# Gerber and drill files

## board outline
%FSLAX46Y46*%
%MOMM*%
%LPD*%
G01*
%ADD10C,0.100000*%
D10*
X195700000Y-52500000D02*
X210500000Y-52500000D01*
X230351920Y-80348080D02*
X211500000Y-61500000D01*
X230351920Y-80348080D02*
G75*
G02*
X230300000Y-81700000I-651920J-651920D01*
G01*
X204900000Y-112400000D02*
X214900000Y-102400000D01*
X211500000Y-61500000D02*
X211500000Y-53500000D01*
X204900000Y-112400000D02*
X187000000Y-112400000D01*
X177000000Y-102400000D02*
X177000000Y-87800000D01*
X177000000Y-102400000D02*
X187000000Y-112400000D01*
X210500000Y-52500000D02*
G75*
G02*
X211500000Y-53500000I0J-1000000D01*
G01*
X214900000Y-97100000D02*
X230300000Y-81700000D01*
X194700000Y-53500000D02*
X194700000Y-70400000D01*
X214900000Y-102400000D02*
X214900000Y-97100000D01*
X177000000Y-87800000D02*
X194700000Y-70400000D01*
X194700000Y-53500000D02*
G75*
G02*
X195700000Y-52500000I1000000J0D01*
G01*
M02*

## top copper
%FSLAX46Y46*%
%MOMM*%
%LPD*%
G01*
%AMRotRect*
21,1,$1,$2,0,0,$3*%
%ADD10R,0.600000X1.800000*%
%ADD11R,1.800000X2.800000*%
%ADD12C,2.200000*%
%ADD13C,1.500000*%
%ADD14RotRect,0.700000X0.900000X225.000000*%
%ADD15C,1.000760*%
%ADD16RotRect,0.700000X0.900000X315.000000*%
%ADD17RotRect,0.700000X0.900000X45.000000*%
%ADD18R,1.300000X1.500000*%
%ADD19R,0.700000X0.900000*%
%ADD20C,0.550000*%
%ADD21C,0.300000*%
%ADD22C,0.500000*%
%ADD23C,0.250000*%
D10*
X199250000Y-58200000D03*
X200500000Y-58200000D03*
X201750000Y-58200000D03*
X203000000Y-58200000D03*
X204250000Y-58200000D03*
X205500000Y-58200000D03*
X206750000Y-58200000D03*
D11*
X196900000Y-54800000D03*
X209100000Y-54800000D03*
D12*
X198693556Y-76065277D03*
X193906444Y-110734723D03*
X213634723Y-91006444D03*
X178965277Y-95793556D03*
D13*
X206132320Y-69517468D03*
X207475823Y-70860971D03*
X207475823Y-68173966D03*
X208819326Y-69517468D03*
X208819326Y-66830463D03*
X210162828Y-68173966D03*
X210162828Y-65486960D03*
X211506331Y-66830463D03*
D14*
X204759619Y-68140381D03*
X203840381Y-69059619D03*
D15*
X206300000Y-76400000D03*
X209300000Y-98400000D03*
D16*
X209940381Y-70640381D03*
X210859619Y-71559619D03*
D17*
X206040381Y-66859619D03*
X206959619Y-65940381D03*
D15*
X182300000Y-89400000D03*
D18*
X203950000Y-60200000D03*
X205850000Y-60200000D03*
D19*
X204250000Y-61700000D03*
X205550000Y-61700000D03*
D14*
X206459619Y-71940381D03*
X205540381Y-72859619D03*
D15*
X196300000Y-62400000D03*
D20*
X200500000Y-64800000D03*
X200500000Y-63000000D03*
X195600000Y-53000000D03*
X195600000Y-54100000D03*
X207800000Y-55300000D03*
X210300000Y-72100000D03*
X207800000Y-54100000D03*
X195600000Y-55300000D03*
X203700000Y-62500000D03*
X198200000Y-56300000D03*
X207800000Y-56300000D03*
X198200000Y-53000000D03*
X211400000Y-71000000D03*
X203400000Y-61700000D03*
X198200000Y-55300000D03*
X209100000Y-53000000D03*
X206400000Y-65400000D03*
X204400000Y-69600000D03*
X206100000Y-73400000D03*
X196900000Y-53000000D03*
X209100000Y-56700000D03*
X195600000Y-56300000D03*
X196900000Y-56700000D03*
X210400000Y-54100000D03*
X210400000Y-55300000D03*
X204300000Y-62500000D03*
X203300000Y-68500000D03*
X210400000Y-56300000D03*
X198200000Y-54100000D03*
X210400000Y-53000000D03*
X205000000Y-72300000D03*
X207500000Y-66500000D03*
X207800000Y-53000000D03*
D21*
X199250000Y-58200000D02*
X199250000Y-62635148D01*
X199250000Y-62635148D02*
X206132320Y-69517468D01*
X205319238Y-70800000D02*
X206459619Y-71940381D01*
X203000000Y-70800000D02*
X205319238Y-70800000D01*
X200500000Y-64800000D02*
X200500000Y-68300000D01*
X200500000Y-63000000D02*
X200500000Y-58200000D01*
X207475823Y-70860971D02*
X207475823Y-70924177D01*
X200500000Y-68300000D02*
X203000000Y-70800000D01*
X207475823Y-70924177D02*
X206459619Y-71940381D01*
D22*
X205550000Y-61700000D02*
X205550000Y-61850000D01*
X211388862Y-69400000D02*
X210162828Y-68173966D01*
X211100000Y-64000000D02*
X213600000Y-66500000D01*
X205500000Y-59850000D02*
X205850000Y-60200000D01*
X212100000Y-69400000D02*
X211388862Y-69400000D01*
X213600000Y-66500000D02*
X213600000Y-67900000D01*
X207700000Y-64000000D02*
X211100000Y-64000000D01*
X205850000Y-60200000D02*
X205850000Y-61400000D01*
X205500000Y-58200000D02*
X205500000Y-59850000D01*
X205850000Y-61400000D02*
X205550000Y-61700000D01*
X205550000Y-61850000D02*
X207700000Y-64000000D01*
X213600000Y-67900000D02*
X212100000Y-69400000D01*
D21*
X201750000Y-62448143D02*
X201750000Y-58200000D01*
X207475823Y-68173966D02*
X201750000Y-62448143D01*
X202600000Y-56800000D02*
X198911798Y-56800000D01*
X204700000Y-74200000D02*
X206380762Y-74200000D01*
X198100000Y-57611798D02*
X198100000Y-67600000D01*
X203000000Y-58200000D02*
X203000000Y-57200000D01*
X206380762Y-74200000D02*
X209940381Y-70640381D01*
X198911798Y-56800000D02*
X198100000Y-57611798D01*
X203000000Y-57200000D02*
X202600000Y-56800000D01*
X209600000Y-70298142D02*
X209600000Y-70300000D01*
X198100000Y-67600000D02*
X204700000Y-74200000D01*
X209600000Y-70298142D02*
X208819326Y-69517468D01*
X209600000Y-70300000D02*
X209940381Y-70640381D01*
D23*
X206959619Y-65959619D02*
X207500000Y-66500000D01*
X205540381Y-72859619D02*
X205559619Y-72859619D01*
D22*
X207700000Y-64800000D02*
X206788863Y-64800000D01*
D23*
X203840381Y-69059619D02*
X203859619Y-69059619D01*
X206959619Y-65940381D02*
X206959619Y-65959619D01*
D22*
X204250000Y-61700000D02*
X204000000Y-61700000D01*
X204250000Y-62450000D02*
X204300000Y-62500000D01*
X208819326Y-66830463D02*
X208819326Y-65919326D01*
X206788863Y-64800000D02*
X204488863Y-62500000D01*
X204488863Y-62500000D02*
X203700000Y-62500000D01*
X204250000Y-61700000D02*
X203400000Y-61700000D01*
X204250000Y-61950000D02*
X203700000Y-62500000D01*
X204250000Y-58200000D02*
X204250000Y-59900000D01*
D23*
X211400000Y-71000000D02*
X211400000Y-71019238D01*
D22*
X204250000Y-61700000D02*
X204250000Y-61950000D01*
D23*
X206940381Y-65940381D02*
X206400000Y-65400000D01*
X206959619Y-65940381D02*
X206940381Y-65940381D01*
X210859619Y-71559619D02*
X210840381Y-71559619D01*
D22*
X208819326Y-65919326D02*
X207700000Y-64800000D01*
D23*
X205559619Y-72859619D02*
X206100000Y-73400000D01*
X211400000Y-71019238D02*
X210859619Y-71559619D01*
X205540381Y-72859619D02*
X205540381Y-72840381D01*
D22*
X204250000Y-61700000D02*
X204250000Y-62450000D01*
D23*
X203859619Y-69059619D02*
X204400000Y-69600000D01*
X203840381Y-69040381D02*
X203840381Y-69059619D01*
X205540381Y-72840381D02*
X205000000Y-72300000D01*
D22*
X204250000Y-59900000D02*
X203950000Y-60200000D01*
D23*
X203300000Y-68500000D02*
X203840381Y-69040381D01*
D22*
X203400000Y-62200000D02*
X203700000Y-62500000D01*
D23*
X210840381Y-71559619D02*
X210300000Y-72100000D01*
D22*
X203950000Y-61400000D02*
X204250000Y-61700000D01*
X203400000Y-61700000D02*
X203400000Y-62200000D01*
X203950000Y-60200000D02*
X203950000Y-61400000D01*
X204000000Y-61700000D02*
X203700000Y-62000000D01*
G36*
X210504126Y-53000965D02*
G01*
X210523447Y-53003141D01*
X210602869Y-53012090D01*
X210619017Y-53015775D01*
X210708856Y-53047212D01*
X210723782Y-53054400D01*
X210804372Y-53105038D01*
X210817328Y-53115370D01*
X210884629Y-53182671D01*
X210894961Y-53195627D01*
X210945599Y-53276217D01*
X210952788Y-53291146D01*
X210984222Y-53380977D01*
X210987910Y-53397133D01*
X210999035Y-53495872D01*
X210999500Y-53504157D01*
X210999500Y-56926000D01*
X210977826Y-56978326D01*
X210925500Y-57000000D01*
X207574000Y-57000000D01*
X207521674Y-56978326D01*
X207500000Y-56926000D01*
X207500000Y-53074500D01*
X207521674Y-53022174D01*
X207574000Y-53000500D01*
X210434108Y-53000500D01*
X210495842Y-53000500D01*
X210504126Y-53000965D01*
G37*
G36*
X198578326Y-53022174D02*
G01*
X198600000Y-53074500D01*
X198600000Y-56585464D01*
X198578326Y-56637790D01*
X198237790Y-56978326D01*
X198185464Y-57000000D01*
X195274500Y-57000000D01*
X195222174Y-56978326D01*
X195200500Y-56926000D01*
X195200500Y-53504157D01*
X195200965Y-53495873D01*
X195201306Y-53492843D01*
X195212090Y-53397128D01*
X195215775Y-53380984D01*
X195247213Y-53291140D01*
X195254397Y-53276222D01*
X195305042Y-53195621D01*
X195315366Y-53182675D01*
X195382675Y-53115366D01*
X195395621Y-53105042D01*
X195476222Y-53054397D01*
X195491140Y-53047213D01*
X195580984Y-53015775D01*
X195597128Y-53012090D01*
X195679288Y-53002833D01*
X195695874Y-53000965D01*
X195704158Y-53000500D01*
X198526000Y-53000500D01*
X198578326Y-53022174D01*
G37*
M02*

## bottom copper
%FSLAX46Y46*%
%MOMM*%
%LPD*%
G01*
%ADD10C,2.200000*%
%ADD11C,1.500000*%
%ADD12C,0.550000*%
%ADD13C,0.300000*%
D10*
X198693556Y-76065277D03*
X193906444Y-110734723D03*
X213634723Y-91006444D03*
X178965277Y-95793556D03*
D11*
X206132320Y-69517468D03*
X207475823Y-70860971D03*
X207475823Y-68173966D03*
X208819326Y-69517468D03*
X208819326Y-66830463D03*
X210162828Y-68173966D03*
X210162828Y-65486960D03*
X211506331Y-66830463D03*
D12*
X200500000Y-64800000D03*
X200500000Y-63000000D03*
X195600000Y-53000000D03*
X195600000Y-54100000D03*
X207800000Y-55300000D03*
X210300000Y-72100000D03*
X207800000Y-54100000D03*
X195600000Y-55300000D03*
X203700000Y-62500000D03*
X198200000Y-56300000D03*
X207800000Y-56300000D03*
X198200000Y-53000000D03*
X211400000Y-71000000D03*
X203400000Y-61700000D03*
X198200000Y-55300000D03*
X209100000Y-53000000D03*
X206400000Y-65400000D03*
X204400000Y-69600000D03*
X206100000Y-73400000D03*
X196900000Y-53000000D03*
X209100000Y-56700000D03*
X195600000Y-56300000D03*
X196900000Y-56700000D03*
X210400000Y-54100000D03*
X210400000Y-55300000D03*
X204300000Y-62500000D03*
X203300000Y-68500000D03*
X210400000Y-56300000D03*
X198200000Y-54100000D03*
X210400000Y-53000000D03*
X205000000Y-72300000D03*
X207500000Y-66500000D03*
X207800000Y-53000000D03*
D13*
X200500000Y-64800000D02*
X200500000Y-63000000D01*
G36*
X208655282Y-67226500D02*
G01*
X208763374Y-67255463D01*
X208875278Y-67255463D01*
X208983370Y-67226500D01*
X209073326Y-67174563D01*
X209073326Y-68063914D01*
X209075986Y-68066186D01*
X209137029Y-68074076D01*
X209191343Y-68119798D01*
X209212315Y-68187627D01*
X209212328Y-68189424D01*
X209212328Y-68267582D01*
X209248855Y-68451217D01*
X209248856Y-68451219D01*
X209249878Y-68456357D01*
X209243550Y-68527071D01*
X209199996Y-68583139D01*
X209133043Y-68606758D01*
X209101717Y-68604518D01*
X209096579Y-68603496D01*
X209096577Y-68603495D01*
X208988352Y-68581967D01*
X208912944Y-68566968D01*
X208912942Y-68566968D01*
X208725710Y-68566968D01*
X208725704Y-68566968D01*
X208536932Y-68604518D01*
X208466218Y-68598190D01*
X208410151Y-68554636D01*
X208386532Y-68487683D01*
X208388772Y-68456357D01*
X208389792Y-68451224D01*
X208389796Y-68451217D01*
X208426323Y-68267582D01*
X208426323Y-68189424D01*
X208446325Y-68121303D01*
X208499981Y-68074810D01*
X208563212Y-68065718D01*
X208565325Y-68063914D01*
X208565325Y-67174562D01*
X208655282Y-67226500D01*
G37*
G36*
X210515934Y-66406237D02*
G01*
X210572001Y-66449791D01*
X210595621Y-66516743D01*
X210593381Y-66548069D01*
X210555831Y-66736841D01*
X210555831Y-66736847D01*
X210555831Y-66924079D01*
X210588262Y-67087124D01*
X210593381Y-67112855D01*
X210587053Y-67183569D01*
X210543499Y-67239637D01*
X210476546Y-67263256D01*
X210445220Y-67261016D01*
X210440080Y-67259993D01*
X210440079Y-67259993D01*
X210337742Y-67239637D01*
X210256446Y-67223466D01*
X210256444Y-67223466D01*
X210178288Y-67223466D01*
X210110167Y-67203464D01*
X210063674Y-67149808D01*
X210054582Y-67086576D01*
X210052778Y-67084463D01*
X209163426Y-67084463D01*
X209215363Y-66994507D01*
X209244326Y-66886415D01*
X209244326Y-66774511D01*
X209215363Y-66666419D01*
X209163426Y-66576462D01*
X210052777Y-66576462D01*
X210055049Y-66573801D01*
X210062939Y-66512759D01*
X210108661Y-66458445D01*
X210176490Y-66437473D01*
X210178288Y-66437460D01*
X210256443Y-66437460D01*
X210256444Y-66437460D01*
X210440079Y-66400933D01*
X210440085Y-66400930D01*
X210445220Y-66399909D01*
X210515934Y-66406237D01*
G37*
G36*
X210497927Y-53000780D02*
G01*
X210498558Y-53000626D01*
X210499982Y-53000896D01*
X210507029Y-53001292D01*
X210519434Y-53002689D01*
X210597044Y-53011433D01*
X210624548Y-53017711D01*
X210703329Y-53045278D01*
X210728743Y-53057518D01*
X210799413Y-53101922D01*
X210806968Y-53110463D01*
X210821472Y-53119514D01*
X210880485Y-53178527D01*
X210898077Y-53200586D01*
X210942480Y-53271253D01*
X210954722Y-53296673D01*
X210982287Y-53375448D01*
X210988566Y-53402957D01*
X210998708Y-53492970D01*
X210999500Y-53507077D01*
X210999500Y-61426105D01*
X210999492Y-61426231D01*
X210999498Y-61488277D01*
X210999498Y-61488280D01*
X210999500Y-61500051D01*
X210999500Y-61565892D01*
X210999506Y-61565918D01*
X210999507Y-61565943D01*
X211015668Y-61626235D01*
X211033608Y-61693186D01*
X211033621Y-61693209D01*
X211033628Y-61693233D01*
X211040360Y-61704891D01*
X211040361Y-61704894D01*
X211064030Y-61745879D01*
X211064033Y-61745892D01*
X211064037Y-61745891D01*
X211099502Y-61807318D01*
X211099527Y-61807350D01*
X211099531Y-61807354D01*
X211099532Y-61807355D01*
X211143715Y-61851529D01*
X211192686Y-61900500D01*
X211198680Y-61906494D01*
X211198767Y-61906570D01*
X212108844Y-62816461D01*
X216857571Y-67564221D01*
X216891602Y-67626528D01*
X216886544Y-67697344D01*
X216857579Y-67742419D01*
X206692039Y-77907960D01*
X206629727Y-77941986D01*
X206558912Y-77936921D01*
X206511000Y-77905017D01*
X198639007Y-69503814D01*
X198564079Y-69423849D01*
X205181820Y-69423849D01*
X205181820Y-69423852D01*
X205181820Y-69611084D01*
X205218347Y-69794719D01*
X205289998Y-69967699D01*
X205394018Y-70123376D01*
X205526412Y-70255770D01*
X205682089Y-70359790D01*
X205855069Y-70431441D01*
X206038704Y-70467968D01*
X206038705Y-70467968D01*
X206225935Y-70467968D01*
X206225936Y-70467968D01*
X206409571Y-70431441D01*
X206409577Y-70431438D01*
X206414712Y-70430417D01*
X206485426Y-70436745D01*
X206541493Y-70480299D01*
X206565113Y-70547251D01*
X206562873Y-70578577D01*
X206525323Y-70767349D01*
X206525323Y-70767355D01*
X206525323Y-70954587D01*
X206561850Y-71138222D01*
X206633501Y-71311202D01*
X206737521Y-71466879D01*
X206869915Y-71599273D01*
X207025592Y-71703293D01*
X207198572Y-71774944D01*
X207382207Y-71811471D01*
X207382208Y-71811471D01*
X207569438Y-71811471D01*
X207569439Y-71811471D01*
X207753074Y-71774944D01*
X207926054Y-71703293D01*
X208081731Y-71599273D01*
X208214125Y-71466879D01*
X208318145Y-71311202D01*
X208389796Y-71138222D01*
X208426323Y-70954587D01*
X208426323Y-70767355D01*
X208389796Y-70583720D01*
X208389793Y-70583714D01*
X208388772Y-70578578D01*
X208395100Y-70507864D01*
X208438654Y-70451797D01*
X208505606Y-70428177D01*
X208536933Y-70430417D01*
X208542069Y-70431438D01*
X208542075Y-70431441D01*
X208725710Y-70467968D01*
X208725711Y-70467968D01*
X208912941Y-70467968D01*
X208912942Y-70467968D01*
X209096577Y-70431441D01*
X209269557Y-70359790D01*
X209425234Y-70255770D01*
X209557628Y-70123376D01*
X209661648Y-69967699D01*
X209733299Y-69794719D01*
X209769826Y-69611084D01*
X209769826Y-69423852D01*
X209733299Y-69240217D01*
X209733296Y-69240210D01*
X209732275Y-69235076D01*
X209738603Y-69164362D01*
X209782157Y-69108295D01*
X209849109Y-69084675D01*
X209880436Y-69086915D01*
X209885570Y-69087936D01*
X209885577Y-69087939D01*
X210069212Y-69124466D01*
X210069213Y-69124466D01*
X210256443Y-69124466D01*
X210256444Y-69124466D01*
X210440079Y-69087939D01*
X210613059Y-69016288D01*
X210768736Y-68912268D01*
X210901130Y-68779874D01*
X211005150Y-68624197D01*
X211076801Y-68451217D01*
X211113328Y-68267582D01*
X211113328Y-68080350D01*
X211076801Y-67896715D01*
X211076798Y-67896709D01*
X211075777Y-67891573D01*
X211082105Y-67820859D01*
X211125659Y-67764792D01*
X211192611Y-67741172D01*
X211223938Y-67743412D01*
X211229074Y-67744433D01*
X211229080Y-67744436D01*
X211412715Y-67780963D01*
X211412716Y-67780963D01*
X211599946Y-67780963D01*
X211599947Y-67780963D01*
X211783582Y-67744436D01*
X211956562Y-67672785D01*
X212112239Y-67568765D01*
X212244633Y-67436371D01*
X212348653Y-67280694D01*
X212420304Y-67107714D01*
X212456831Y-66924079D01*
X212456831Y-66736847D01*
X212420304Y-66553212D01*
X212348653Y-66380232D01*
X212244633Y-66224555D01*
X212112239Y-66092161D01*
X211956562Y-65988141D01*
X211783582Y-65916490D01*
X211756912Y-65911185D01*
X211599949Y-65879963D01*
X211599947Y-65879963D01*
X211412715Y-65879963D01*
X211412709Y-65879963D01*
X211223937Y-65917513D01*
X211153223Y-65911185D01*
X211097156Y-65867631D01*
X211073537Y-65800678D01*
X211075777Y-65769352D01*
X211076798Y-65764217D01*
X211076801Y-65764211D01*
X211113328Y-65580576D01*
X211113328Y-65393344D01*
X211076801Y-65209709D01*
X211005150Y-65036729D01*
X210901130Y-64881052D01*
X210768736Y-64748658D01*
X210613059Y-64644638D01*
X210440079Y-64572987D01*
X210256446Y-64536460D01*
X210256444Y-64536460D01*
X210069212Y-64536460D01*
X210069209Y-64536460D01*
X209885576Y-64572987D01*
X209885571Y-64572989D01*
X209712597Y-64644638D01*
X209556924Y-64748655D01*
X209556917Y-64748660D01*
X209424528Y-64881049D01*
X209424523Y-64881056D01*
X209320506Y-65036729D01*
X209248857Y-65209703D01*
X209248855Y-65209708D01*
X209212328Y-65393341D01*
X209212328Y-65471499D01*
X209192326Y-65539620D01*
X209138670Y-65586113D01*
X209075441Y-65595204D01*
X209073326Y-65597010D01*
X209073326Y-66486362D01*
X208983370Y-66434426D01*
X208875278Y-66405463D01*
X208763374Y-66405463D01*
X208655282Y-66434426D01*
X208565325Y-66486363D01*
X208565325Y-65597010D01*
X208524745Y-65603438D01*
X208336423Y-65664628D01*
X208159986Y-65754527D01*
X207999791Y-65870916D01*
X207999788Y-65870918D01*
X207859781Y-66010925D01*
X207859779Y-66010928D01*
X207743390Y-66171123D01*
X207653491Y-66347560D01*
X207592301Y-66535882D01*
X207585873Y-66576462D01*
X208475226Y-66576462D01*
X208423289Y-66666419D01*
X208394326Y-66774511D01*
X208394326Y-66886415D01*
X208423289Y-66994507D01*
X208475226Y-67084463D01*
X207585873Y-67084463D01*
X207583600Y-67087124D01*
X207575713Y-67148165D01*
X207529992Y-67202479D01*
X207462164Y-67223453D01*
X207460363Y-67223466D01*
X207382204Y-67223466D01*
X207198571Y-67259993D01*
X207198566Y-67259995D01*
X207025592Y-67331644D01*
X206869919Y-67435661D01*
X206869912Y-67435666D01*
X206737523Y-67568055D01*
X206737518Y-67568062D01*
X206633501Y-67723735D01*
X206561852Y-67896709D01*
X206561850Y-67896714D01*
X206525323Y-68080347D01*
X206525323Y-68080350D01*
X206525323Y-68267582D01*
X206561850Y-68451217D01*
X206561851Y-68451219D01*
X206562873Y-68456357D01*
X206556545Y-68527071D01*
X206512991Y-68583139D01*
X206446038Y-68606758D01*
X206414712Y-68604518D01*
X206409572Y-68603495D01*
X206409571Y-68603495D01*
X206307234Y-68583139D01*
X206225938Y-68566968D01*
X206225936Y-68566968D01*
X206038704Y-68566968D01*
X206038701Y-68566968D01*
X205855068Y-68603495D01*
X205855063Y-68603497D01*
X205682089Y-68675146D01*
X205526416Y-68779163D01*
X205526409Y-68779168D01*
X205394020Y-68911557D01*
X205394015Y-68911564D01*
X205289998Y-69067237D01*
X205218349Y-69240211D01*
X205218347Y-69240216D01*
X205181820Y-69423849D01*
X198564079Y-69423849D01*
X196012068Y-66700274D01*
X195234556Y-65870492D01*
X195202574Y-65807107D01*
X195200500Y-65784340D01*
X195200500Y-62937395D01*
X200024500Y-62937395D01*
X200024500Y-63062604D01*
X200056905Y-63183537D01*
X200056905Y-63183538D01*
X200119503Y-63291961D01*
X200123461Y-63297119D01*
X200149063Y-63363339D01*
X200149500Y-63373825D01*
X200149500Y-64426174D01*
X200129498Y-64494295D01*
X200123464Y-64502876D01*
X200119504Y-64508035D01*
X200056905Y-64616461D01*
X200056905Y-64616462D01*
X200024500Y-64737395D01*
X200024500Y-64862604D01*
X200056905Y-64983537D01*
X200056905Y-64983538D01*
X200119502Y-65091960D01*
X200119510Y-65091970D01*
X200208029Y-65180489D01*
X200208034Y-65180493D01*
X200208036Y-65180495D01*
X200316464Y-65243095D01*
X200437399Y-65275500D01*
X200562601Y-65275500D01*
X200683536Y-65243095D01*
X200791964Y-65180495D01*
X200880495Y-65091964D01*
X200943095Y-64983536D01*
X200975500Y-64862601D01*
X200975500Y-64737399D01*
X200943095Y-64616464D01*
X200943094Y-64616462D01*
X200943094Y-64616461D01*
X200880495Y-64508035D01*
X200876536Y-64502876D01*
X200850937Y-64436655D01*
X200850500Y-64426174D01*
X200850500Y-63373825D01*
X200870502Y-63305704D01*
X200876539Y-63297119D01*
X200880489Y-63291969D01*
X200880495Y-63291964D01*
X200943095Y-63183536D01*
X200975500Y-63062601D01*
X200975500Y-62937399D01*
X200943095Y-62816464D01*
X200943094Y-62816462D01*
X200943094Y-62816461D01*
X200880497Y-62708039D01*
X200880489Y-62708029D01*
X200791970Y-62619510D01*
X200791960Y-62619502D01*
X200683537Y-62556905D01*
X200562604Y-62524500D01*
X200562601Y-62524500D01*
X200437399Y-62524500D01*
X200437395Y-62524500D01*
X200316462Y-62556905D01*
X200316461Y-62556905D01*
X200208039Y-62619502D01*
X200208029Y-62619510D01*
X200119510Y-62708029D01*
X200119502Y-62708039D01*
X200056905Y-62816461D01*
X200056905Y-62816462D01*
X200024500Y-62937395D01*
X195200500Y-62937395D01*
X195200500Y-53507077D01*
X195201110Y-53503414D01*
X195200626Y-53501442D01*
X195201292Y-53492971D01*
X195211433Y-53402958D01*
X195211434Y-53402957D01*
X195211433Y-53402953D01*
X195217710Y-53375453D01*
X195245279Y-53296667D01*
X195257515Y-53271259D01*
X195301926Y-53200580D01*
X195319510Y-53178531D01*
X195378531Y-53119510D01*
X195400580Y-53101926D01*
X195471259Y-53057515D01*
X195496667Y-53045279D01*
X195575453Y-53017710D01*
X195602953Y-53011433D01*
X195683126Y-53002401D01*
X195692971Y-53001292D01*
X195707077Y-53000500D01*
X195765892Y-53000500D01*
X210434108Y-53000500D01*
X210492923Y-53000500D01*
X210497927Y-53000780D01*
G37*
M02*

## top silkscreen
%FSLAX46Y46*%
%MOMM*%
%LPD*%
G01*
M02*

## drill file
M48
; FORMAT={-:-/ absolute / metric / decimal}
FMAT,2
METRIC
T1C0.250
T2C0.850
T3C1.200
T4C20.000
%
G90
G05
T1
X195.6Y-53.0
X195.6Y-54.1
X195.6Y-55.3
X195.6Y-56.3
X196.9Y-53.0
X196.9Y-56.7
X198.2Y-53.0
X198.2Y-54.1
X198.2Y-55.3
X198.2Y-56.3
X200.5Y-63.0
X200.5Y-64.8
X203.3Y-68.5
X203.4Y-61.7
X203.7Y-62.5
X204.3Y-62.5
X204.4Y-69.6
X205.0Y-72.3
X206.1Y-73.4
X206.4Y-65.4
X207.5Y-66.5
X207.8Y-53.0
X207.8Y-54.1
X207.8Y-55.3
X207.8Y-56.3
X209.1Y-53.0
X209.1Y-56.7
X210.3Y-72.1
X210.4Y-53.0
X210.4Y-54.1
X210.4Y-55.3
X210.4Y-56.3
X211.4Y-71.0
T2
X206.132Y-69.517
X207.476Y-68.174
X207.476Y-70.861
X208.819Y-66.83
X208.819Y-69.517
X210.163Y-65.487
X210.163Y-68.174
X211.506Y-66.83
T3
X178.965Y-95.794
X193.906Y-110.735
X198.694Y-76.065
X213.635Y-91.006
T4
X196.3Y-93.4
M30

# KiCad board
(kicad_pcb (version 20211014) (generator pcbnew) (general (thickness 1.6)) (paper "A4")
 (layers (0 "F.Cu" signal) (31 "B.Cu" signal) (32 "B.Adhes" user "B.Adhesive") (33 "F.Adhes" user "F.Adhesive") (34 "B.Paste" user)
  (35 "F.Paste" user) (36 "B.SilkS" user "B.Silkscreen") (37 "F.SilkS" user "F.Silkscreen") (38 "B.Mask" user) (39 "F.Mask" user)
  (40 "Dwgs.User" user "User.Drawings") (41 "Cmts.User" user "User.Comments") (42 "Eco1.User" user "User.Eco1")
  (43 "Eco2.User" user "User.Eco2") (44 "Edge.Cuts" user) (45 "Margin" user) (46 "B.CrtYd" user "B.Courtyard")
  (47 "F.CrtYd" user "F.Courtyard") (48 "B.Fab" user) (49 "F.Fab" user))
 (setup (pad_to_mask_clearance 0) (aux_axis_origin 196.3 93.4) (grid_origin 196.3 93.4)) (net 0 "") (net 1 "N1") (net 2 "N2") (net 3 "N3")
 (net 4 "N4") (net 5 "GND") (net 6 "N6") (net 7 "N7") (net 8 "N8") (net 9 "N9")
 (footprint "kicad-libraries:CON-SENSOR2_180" (layer "F.Cu") (at 203 53.4 180)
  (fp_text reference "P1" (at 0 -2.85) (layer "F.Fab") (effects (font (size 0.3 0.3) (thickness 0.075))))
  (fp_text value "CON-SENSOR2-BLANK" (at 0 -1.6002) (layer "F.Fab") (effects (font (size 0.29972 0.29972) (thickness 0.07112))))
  (pad "1" smd rect locked (at 3.75 -4.8 180) (size 0.6 1.8) (layers "F.Cu" "F.Paste" "F.Mask") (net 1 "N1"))
  (pad "2" smd rect locked (at 2.5 -4.8 180) (size 0.6 1.8) (layers "F.Cu" "F.Paste" "F.Mask") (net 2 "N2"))
  (pad "3" smd rect locked (at 1.25 -4.8 180) (size 0.6 1.8) (layers "F.Cu" "F.Paste" "F.Mask") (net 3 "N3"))
  (pad "4" smd rect locked (at 0 -4.8 180) (size 0.6 1.8) (layers "F.Cu" "F.Paste" "F.Mask") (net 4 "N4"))
  (pad "5" smd rect locked (at -1.25 -4.8 180) (size 0.6 1.8) (layers "F.Cu" "F.Paste" "F.Mask") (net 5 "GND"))
  (pad "6" smd rect locked (at -2.5 -4.8 180) (size 0.6 1.8) (layers "F.Cu" "F.Paste" "F.Mask") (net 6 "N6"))
  (pad "7" smd rect locked (at -3.75 -4.8 180) (size 0.6 1.8) (layers "F.Cu" "F.Paste" "F.Mask") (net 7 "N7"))
  (pad "EP" smd rect locked (at 6.1 -1.4 180) (size 1.8 2.8) (layers "F.Cu" "F.Paste" "F.Mask") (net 5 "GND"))
  (pad "EP" smd rect locked (at -6.1 -1.4 180) (size 1.8 2.8) (layers "F.Cu" "F.Paste" "F.Mask") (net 5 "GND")))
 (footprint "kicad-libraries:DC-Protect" (layer "F.Cu") (at 196.3 93.4 135)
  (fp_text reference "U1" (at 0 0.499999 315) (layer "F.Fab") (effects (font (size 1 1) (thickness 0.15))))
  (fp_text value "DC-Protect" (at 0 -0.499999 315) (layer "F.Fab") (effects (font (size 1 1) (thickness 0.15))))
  (pad "" thru_hole circle locked (at 10.565 13.95 135) (size 2.2 2.2) (drill 1.2) (layers *.Cu *.Mask))
  (pad "" thru_hole circle locked (at -10.565 -13.95 135) (size 2.2 2.2) (drill 1.2) (layers *.Cu *.Mask))
  (pad "" thru_hole circle locked (at -10.565 13.95 135) (size 2.2 2.2) (drill 1.2) (layers *.Cu *.Mask))
  (pad "" thru_hole circle locked (at 10.565 -13.95 135) (size 2.2 2.2) (drill 1.2) (layers *.Cu *.Mask))
  (pad "" np_thru_hole circle locked (at 0 0 135) (size 20 20) (drill 20) (layers *.Cu *.Mask))
  (pad "1" thru_hole circle locked (at 9.935 23.84 135) (size 1.5 1.5) (drill 0.85) (layers *.Cu *.Mask) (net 1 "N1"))
  (pad "2" thru_hole circle locked (at 8.035 23.84 135) (size 1.5 1.5) (drill 0.85) (layers *.Cu *.Mask) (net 2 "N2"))
  (pad "3" thru_hole circle locked (at 9.935 25.74 135) (size 1.5 1.5) (drill 0.85) (layers *.Cu *.Mask) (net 3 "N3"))
  (pad "4" thru_hole circle locked (at 8.035 25.74 135) (size 1.5 1.5) (drill 0.85) (layers *.Cu *.Mask) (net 4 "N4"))
  (pad "5" thru_hole circle locked (at 9.935 27.64 135) (size 1.5 1.5) (drill 0.85) (layers *.Cu *.Mask) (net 5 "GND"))
  (pad "6" thru_hole circle locked (at 8.035 27.64 135) (size 1.5 1.5) (drill 0.85) (layers *.Cu *.Mask) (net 6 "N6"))
  (pad "7" thru_hole circle locked (at 9.935 29.54 135) (size 1.5 1.5) (drill 0.85) (layers *.Cu *.Mask) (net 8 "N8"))
  (pad "8" thru_hole circle locked (at 8.035 29.54 135) (size 1.5 1.5) (drill 0.85) (layers *.Cu *.Mask) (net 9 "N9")))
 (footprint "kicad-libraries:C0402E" (layer "F.Cu") (at 204.3 68.6 -135)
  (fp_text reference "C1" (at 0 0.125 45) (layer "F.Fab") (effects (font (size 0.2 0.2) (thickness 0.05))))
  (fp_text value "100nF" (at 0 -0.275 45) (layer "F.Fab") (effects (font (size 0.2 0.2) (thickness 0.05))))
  (pad "1" smd rect locked (at -0.65 0 225) (size 0.7 0.9) (layers "F.Cu" "F.Paste" "F.Mask") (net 1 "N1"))
  (pad "2" smd rect locked (at 0.65 0 225) (size 0.7 0.9) (layers "F.Cu" "F.Paste" "F.Mask") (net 5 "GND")))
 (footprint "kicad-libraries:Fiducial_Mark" (layer "F.Cu") (at 206.3 76.4)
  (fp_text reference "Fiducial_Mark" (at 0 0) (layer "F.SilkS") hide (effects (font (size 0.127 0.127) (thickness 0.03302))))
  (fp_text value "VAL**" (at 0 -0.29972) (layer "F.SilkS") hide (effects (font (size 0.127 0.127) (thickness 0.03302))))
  (pad "1" smd circle locked (at 0 0) (size 1.00076 1.00076) (layers "F.Cu" "F.Paste" "F.Mask") (clearance 0.65024)))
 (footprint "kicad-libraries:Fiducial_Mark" (layer "F.Cu") (at 209.3 98.4)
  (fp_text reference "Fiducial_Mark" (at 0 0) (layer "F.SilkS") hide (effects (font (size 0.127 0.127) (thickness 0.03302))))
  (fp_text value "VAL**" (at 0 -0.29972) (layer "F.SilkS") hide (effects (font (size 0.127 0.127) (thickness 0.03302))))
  (pad "1" smd circle locked (at 0 0) (size 1.00076 1.00076) (layers "F.Cu" "F.Paste" "F.Mask") (clearance 0.65024)))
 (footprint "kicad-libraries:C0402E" (layer "F.Cu") (at 210.4 71.1 -45)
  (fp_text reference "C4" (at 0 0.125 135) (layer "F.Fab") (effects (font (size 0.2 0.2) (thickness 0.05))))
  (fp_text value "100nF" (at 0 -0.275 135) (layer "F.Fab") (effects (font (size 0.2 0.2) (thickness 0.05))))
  (pad "1" smd rect locked (at -0.65 0 315) (size 0.7 0.9) (layers "F.Cu" "F.Paste" "F.Mask") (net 4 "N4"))
  (pad "2" smd rect locked (at 0.65 0 315) (size 0.7 0.9) (layers "F.Cu" "F.Paste" "F.Mask") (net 5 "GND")))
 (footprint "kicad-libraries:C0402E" (layer "F.Cu") (at 206.5 66.4 45)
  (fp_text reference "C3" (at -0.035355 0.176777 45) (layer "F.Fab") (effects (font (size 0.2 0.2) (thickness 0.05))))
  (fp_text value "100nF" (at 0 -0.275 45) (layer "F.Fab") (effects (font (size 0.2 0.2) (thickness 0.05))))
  (pad "1" smd rect locked (at -0.65 0 45) (size 0.7 0.9) (layers "F.Cu" "F.Paste" "F.Mask") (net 3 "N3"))
  (pad "2" smd rect locked (at 0.65 0 45) (size 0.7 0.9) (layers "F.Cu" "F.Paste" "F.Mask") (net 5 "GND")))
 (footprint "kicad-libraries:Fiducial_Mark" (layer "F.Cu") (at 182.3 89.4)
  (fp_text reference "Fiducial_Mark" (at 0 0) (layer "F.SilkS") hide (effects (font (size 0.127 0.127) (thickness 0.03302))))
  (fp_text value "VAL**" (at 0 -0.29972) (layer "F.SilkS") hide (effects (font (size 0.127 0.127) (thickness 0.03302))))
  (pad "1" smd circle locked (at 0 0) (size 1.00076 1.00076) (layers "F.Cu" "F.Paste" "F.Mask") (clearance 0.65024)))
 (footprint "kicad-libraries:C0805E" (layer "F.Cu") (at 204.9 60.2)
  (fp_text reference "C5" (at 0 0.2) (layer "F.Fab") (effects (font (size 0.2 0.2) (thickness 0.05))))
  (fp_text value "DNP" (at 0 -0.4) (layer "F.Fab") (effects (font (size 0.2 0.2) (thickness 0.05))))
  (pad "1" smd rect locked (at -0.95 0) (size 1.3 1.5) (layers "F.Cu" "F.Paste" "F.Mask") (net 5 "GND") (clearance 0.14986))
  (pad "2" smd rect locked (at 0.95 0) (size 1.3 1.5) (layers "F.Cu" "F.Paste" "F.Mask") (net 6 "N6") (clearance 0.14986)))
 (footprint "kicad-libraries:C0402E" (layer "F.Cu") (at 204.9 61.7)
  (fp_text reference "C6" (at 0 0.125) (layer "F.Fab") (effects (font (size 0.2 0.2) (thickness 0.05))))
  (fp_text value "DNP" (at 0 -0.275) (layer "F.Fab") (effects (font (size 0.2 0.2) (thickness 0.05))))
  (pad "1" smd rect locked (at -0.65 0) (size 0.7 0.9) (layers "F.Cu" "F.Paste" "F.Mask") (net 5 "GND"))
  (pad "2" smd rect locked (at 0.65 0) (size 0.7 0.9) (layers "F.Cu" "F.Paste" "F.Mask") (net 6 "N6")))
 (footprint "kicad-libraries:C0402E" (layer "F.Cu") (at 206 72.4 -135)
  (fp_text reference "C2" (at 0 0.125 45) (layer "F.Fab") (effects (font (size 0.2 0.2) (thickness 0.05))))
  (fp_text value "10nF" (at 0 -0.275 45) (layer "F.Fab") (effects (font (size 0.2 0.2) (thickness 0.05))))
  (pad "1" smd rect locked (at -0.65 0 225) (size 0.7 0.9) (layers "F.Cu" "F.Paste" "F.Mask") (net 2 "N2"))
  (pad "2" smd rect locked (at 0.65 0 225) (size 0.7 0.9) (layers "F.Cu" "F.Paste" "F.Mask") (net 5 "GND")))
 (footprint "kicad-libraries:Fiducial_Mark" (layer "F.Cu") (at 196.3 62.4)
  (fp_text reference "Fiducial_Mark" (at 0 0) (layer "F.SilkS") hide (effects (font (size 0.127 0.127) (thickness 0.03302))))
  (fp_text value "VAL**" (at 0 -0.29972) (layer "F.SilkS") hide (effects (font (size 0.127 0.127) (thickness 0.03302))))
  (pad "1" smd circle locked (at 0 0) (size 1.00076 1.00076) (layers "F.Cu" "F.Paste" "F.Mask") (clearance 0.65024)))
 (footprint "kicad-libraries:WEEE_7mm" (layer "B.Cu") (at 188.8 106.4 180)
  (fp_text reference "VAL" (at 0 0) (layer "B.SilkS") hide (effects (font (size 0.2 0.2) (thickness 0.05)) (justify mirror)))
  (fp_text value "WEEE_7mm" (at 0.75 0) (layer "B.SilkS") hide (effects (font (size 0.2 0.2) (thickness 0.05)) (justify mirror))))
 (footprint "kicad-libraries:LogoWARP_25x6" (layer "B.Cu") (at 213.6 81 180)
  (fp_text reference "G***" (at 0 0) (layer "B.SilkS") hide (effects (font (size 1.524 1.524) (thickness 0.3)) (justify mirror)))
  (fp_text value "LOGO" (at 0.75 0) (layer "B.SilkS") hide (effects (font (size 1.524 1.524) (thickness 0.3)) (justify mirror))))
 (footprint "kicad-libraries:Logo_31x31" (layer "B.Cu") (at 201.4 105.1 180)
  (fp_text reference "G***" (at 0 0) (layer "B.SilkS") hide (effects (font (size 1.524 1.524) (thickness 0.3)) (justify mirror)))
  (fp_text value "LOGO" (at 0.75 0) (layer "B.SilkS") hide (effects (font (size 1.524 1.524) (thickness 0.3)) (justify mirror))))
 (gr_line (start 195.7 52.5) (end 210.5 52.5) (layer "Edge.Cuts") (width 0.1))
 (gr_line (start 230.35192 80.34808) (end 211.5 61.5) (layer "Edge.Cuts") (width 0.1))
 (gr_arc (start 230.35192 80.34808) (mid 230.621275 81.035381) (end 230.3 81.7) (layer "Edge.Cuts") (width 0.1))
 (gr_line (start 204.9 112.4) (end 214.9 102.4) (layer "Edge.Cuts") (width 0.1))
 (gr_line (start 211.5 61.5) (end 211.5 53.5) (layer "Edge.Cuts") (width 0.1))
 (gr_line (start 204.9 112.4) (end 187 112.4) (layer "Edge.Cuts") (width 0.1))
 (gr_line (start 177 102.4) (end 177 87.8) (layer "Edge.Cuts") (width 0.1))
 (gr_line (start 177 102.4) (end 187 112.4) (layer "Edge.Cuts") (width 0.1))
 (gr_arc (start 210.5 52.5) (mid 211.207107 52.792893) (end 211.5 53.5) (layer "Edge.Cuts") (width 0.1))
 (gr_line (start 214.9 97.1) (end 230.3 81.7) (layer "Edge.Cuts") (width 0.1))
 (gr_line (start 194.7 53.5) (end 194.7 70.4) (layer "Edge.Cuts") (width 0.1))
 (gr_line (start 214.9 102.4) (end 214.9 97.1) (layer "Edge.Cuts") (width 0.1))
 (gr_line (start 177 87.8) (end 194.7 70.4) (layer "Edge.Cuts") (width 0.1))
 (gr_arc (start 194.7 53.5) (mid 194.992893 52.792893) (end 195.7 52.5) (layer "Edge.Cuts") (width 0.1))
 (segment (start 199.25 58.2) (end 199.25 62.635148) (width 0.3) (layer "F.Cu") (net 1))
 (segment (start 199.25 62.635148) (end 206.13232 69.517468) (width 0.3) (layer "F.Cu") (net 1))
 (segment (start 205.319238 70.8) (end 206.459619 71.940381) (width 0.3) (layer "F.Cu") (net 2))
 (segment (start 203 70.8) (end 205.319238 70.8) (width 0.3) (layer "F.Cu") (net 2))
 (segment (start 200.5 64.8) (end 200.5 68.3) (width 0.3) (layer "F.Cu") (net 2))
 (segment (start 200.5 63) (end 200.5 58.2) (width 0.3) (layer "F.Cu") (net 2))
 (segment (start 207.475823 70.860971) (end 207.475823 70.924177) (width 0.3) (layer "F.Cu") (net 2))
 (segment (start 200.5 68.3) (end 203 70.8) (width 0.3) (layer "F.Cu") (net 2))
 (segment (start 207.475823 70.924177) (end 206.459619 71.940381) (width 0.3) (layer "F.Cu") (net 2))
 (via (at 200.5 64.8) (size 0.55) (drill 0.25) (layers "F.Cu" "B.Cu") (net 2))
 (via (at 200.5 63) (size 0.55) (drill 0.25) (layers "F.Cu" "B.Cu") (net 2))
 (segment (start 200.5 64.8) (end 200.5 63) (width 0.3) (layer "B.Cu") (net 2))
 (segment (start 205.55 61.7) (end 205.55 61.85) (width 0.5) (layer "F.Cu") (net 6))
 (segment (start 211.388862 69.4) (end 210.162828 68.173966) (width 0.5) (layer "F.Cu") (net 6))
 (segment (start 211.1 64) (end 213.6 66.5) (width 0.5) (layer "F.Cu") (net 6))
 (segment (start 205.5 59.85) (end 205.85 60.2) (width 0.5) (layer "F.Cu") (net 6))
 (segment (start 212.1 69.4) (end 211.388862 69.4) (width 0.5) (layer "F.Cu") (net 6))
 (segment (start 213.6 66.5) (end 213.6 67.9) (width 0.5) (layer "F.Cu") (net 6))
 (segment (start 207.7 64) (end 211.1 64) (width 0.5) (layer "F.Cu") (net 6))
 (segment (start 205.85 60.2) (end 205.85 61.4) (width 0.5) (layer "F.Cu") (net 6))
 (segment (start 205.5 58.2) (end 205.5 59.85) (width 0.5) (layer "F.Cu") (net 6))
 (segment (start 205.85 61.4) (end 205.55 61.7) (width 0.5) (layer "F.Cu") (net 6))
 (segment (start 205.55 61.85) (end 207.7 64) (width 0.5) (layer "F.Cu") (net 6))
 (segment (start 213.6 67.9) (end 212.1 69.4) (width 0.5) (layer "F.Cu") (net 6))
 (segment (start 201.75 62.448143) (end 201.75 58.2) (width 0.3) (layer "F.Cu") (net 3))
 (segment (start 207.475823 68.173966) (end 201.75 62.448143) (width 0.3) (layer "F.Cu") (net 3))
 (segment (start 202.6 56.8) (end 198.911798 56.8) (width 0.3) (layer "F.Cu") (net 4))
 (segment (start 204.7 74.2) (end 206.380762 74.2) (width 0.3) (layer "F.Cu") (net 4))
 (segment (start 198.1 57.611798) (end 198.1 67.6) (width 0.3) (layer "F.Cu") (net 4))
 (segment (start 203 58.2) (end 203 57.2) (width 0.3) (layer "F.Cu") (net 4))
 (segment (start 206.380762 74.2) (end 209.940381 70.640381) (width 0.3) (layer "F.Cu") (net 4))
 (segment (start 198.911798 56.8) (end 198.1 57.611798) (width 0.3) (layer "F.Cu") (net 4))
 (segment (start 203 57.2) (end 202.6 56.8) (width 0.3) (layer "F.Cu") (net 4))
 (segment (start 209.6 70.298142) (end 209.6 70.3) (width 0.3) (layer "F.Cu") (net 4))
 (segment (start 198.1 67.6) (end 204.7 74.2) (width 0.3) (layer "F.Cu") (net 4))
 (segment (start 209.6 70.298142) (end 208.819326 69.517468) (width 0.3) (layer "F.Cu") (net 4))
 (segment (start 209.6 70.3) (end 209.940381 70.640381) (width 0.3) (layer "F.Cu") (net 4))
 (segment (start 206.959619 65.959619) (end 207.5 66.5) (width 0.25) (layer "F.Cu") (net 5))
 (segment (start 205.540381 72.859619) (end 205.559619 72.859619) (width 0.25) (layer "F.Cu") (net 5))
 (segment (start 207.7 64.8) (end 206.788863 64.8) (width 0.5) (layer "F.Cu") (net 5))
 (segment (start 203.840381 69.059619) (end 203.859619 69.059619) (width 0.25) (layer "F.Cu") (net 5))
 (segment (start 206.959619 65.940381) (end 206.959619 65.959619) (width 0.25) (layer "F.Cu") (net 5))
 (segment (start 204.25 61.7) (end 204 61.7) (width 0.5) (layer "F.Cu") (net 5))
 (segment (start 204.25 62.45) (end 204.3 62.5) (width 0.5) (layer "F.Cu") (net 5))
 (segment (start 208.819326 66.830463) (end 208.819326 65.919326) (width 0.5) (layer "F.Cu") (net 5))
 (segment (start 206.788863 64.8) (end 204.488863 62.5) (width 0.5) (layer "F.Cu") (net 5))
 (segment (start 204.488863 62.5) (end 203.7 62.5) (width 0.5) (layer "F.Cu") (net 5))
 (segment (start 204.25 61.7) (end 203.4 61.7) (width 0.5) (layer "F.Cu") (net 5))
 (segment (start 204.25 61.95) (end 203.7 62.5) (width 0.5) (layer "F.Cu") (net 5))
 (segment (start 204.25 58.2) (end 204.25 59.9) (width 0.5) (layer "F.Cu") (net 5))
 (segment (start 211.4 71) (end 211.4 71.019238) (width 0.25) (layer "F.Cu") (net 5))
 (segment (start 204.25 61.7) (end 204.25 61.95) (width 0.5) (layer "F.Cu") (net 5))
 (segment (start 206.940381 65.940381) (end 206.4 65.4) (width 0.25) (layer "F.Cu") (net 5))
 (segment (start 206.959619 65.940381) (end 206.940381 65.940381) (width 0.25) (layer "F.Cu") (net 5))
 (segment (start 210.859619 71.559619) (end 210.840381 71.559619) (width 0.25) (layer "F.Cu") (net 5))
 (segment (start 208.819326 65.919326) (end 207.7 64.8) (width 0.5) (layer "F.Cu") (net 5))
 (segment (start 205.559619 72.859619) (end 206.1 73.4) (width 0.25) (layer "F.Cu") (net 5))
 (segment (start 211.4 71.019238) (end 210.859619 71.559619) (width 0.25) (layer "F.Cu") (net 5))
 (segment (start 205.540381 72.859619) (end 205.540381 72.840381) (width 0.25) (layer "F.Cu") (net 5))
 (segment (start 204.25 61.7) (end 204.25 62.45) (width 0.5) (layer "F.Cu") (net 5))
 (segment (start 203.859619 69.059619) (end 204.4 69.6) (width 0.25) (layer "F.Cu") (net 5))
 (segment (start 203.840381 69.040381) (end 203.840381 69.059619) (width 0.25) (layer "F.Cu") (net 5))
 (segment (start 205.540381 72.840381) (end 205 72.3) (width 0.25) (layer "F.Cu") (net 5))
 (segment (start 204.25 59.9) (end 203.95 60.2) (width 0.5) (layer "F.Cu") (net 5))
 (segment (start 203.3 68.5) (end 203.840381 69.040381) (width 0.25) (layer "F.Cu") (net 5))
 (segment (start 203.4 62.2) (end 203.7 62.5) (width 0.5) (layer "F.Cu") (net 5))
 (segment (start 210.840381 71.559619) (end 210.3 72.1) (width 0.25) (layer "F.Cu") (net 5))
 (segment (start 203.95 61.4) (end 204.25 61.7) (width 0.5) (layer "F.Cu") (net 5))
 (segment (start 203.4 61.7) (end 203.4 62.2) (width 0.5) (layer "F.Cu") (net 5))
 (segment (start 203.95 60.2) (end 203.95 61.4) (width 0.5) (layer "F.Cu") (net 5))
 (segment (start 204 61.7) (end 203.7 62) (width 0.5) (layer "F.Cu") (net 5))
 (via (at 195.6 53) (size 0.55) (drill 0.25) (layers "F.Cu" "B.Cu") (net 5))
 (via (at 195.6 54.1) (size 0.55) (drill 0.25) (layers "F.Cu" "B.Cu") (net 5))
 (via (at 207.8 55.3) (size 0.55) (drill 0.25) (layers "F.Cu" "B.Cu") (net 5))
 (via (at 210.3 72.1) (size 0.55) (drill 0.25) (layers "F.Cu" "B.Cu") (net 5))
 (via (at 207.8 54.1) (size 0.55) (drill 0.25) (layers "F.Cu" "B.Cu") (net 5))
 (via (at 195.6 55.3) (size 0.55) (drill 0.25) (layers "F.Cu" "B.Cu") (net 5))
 (via (at 203.7 62.5) (size 0.55) (drill 0.25) (layers "F.Cu" "B.Cu") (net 5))
 (via (at 198.2 56.3) (size 0.55) (drill 0.25) (layers "F.Cu" "B.Cu") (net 5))
 (via (at 207.8 56.3) (size 0.55) (drill 0.25) (layers "F.Cu" "B.Cu") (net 5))
 (via (at 198.2 53) (size 0.55) (drill 0.25) (layers "F.Cu" "B.Cu") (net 5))
 (via (at 211.4 71) (size 0.55) (drill 0.25) (layers "F.Cu" "B.Cu") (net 5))
 (via (at 203.4 61.7) (size 0.55) (drill 0.25) (layers "F.Cu" "B.Cu") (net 5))
 (via (at 198.2 55.3) (size 0.55) (drill 0.25) (layers "F.Cu" "B.Cu") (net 5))
 (via (at 209.1 53) (size 0.55) (drill 0.25) (layers "F.Cu" "B.Cu") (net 5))
 (via (at 206.4 65.4) (size 0.55) (drill 0.25) (layers "F.Cu" "B.Cu") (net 5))
 (via (at 204.4 69.6) (size 0.55) (drill 0.25) (layers "F.Cu" "B.Cu") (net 5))
 (via (at 206.1 73.4) (size 0.55) (drill 0.25) (layers "F.Cu" "B.Cu") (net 5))
 (via (at 196.9 53) (size 0.55) (drill 0.25) (layers "F.Cu" "B.Cu") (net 5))
 (via (at 209.1 56.7) (size 0.55) (drill 0.25) (layers "F.Cu" "B.Cu") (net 5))
 (via (at 195.6 56.3) (size 0.55) (drill 0.25) (layers "F.Cu" "B.Cu") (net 5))
 (via (at 196.9 56.7) (size 0.55) (drill 0.25) (layers "F.Cu" "B.Cu") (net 5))
 (via (at 210.4 54.1) (size 0.55) (drill 0.25) (layers "F.Cu" "B.Cu") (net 5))
 (via (at 210.4 55.3) (size 0.55) (drill 0.25) (layers "F.Cu" "B.Cu") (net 5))
 (via (at 204.3 62.5) (size 0.55) (drill 0.25) (layers "F.Cu" "B.Cu") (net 5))
 (via (at 203.3 68.5) (size 0.55) (drill 0.25) (layers "F.Cu" "B.Cu") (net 5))
 (via (at 210.4 56.3) (size 0.55) (drill 0.25) (layers "F.Cu" "B.Cu") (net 5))
 (via (at 198.2 54.1) (size 0.55) (drill 0.25) (layers "F.Cu" "B.Cu") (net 5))
 (via (at 210.4 53) (size 0.55) (drill 0.25) (layers "F.Cu" "B.Cu") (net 5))
 (via (at 205 72.3) (size 0.55) (drill 0.25) (layers "F.Cu" "B.Cu") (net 5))
 (via (at 207.5 66.5) (size 0.55) (drill 0.25) (layers "F.Cu" "B.Cu") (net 5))
 (via (at 207.8 53) (size 0.55) (drill 0.25) (layers "F.Cu" "B.Cu") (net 5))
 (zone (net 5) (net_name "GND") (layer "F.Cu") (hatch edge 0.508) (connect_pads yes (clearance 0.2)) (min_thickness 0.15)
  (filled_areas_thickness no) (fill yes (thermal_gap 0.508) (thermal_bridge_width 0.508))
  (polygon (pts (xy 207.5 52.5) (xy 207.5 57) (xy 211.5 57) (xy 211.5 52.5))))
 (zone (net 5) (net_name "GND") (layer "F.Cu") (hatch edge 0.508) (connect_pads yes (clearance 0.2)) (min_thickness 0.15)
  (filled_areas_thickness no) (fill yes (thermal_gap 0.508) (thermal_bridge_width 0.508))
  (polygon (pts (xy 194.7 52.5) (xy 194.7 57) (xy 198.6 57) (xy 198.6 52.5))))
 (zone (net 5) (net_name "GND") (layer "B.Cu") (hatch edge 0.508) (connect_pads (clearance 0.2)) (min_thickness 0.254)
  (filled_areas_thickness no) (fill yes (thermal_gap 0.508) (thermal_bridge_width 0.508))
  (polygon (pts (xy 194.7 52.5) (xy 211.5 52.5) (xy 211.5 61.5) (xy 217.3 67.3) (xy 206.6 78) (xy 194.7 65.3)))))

